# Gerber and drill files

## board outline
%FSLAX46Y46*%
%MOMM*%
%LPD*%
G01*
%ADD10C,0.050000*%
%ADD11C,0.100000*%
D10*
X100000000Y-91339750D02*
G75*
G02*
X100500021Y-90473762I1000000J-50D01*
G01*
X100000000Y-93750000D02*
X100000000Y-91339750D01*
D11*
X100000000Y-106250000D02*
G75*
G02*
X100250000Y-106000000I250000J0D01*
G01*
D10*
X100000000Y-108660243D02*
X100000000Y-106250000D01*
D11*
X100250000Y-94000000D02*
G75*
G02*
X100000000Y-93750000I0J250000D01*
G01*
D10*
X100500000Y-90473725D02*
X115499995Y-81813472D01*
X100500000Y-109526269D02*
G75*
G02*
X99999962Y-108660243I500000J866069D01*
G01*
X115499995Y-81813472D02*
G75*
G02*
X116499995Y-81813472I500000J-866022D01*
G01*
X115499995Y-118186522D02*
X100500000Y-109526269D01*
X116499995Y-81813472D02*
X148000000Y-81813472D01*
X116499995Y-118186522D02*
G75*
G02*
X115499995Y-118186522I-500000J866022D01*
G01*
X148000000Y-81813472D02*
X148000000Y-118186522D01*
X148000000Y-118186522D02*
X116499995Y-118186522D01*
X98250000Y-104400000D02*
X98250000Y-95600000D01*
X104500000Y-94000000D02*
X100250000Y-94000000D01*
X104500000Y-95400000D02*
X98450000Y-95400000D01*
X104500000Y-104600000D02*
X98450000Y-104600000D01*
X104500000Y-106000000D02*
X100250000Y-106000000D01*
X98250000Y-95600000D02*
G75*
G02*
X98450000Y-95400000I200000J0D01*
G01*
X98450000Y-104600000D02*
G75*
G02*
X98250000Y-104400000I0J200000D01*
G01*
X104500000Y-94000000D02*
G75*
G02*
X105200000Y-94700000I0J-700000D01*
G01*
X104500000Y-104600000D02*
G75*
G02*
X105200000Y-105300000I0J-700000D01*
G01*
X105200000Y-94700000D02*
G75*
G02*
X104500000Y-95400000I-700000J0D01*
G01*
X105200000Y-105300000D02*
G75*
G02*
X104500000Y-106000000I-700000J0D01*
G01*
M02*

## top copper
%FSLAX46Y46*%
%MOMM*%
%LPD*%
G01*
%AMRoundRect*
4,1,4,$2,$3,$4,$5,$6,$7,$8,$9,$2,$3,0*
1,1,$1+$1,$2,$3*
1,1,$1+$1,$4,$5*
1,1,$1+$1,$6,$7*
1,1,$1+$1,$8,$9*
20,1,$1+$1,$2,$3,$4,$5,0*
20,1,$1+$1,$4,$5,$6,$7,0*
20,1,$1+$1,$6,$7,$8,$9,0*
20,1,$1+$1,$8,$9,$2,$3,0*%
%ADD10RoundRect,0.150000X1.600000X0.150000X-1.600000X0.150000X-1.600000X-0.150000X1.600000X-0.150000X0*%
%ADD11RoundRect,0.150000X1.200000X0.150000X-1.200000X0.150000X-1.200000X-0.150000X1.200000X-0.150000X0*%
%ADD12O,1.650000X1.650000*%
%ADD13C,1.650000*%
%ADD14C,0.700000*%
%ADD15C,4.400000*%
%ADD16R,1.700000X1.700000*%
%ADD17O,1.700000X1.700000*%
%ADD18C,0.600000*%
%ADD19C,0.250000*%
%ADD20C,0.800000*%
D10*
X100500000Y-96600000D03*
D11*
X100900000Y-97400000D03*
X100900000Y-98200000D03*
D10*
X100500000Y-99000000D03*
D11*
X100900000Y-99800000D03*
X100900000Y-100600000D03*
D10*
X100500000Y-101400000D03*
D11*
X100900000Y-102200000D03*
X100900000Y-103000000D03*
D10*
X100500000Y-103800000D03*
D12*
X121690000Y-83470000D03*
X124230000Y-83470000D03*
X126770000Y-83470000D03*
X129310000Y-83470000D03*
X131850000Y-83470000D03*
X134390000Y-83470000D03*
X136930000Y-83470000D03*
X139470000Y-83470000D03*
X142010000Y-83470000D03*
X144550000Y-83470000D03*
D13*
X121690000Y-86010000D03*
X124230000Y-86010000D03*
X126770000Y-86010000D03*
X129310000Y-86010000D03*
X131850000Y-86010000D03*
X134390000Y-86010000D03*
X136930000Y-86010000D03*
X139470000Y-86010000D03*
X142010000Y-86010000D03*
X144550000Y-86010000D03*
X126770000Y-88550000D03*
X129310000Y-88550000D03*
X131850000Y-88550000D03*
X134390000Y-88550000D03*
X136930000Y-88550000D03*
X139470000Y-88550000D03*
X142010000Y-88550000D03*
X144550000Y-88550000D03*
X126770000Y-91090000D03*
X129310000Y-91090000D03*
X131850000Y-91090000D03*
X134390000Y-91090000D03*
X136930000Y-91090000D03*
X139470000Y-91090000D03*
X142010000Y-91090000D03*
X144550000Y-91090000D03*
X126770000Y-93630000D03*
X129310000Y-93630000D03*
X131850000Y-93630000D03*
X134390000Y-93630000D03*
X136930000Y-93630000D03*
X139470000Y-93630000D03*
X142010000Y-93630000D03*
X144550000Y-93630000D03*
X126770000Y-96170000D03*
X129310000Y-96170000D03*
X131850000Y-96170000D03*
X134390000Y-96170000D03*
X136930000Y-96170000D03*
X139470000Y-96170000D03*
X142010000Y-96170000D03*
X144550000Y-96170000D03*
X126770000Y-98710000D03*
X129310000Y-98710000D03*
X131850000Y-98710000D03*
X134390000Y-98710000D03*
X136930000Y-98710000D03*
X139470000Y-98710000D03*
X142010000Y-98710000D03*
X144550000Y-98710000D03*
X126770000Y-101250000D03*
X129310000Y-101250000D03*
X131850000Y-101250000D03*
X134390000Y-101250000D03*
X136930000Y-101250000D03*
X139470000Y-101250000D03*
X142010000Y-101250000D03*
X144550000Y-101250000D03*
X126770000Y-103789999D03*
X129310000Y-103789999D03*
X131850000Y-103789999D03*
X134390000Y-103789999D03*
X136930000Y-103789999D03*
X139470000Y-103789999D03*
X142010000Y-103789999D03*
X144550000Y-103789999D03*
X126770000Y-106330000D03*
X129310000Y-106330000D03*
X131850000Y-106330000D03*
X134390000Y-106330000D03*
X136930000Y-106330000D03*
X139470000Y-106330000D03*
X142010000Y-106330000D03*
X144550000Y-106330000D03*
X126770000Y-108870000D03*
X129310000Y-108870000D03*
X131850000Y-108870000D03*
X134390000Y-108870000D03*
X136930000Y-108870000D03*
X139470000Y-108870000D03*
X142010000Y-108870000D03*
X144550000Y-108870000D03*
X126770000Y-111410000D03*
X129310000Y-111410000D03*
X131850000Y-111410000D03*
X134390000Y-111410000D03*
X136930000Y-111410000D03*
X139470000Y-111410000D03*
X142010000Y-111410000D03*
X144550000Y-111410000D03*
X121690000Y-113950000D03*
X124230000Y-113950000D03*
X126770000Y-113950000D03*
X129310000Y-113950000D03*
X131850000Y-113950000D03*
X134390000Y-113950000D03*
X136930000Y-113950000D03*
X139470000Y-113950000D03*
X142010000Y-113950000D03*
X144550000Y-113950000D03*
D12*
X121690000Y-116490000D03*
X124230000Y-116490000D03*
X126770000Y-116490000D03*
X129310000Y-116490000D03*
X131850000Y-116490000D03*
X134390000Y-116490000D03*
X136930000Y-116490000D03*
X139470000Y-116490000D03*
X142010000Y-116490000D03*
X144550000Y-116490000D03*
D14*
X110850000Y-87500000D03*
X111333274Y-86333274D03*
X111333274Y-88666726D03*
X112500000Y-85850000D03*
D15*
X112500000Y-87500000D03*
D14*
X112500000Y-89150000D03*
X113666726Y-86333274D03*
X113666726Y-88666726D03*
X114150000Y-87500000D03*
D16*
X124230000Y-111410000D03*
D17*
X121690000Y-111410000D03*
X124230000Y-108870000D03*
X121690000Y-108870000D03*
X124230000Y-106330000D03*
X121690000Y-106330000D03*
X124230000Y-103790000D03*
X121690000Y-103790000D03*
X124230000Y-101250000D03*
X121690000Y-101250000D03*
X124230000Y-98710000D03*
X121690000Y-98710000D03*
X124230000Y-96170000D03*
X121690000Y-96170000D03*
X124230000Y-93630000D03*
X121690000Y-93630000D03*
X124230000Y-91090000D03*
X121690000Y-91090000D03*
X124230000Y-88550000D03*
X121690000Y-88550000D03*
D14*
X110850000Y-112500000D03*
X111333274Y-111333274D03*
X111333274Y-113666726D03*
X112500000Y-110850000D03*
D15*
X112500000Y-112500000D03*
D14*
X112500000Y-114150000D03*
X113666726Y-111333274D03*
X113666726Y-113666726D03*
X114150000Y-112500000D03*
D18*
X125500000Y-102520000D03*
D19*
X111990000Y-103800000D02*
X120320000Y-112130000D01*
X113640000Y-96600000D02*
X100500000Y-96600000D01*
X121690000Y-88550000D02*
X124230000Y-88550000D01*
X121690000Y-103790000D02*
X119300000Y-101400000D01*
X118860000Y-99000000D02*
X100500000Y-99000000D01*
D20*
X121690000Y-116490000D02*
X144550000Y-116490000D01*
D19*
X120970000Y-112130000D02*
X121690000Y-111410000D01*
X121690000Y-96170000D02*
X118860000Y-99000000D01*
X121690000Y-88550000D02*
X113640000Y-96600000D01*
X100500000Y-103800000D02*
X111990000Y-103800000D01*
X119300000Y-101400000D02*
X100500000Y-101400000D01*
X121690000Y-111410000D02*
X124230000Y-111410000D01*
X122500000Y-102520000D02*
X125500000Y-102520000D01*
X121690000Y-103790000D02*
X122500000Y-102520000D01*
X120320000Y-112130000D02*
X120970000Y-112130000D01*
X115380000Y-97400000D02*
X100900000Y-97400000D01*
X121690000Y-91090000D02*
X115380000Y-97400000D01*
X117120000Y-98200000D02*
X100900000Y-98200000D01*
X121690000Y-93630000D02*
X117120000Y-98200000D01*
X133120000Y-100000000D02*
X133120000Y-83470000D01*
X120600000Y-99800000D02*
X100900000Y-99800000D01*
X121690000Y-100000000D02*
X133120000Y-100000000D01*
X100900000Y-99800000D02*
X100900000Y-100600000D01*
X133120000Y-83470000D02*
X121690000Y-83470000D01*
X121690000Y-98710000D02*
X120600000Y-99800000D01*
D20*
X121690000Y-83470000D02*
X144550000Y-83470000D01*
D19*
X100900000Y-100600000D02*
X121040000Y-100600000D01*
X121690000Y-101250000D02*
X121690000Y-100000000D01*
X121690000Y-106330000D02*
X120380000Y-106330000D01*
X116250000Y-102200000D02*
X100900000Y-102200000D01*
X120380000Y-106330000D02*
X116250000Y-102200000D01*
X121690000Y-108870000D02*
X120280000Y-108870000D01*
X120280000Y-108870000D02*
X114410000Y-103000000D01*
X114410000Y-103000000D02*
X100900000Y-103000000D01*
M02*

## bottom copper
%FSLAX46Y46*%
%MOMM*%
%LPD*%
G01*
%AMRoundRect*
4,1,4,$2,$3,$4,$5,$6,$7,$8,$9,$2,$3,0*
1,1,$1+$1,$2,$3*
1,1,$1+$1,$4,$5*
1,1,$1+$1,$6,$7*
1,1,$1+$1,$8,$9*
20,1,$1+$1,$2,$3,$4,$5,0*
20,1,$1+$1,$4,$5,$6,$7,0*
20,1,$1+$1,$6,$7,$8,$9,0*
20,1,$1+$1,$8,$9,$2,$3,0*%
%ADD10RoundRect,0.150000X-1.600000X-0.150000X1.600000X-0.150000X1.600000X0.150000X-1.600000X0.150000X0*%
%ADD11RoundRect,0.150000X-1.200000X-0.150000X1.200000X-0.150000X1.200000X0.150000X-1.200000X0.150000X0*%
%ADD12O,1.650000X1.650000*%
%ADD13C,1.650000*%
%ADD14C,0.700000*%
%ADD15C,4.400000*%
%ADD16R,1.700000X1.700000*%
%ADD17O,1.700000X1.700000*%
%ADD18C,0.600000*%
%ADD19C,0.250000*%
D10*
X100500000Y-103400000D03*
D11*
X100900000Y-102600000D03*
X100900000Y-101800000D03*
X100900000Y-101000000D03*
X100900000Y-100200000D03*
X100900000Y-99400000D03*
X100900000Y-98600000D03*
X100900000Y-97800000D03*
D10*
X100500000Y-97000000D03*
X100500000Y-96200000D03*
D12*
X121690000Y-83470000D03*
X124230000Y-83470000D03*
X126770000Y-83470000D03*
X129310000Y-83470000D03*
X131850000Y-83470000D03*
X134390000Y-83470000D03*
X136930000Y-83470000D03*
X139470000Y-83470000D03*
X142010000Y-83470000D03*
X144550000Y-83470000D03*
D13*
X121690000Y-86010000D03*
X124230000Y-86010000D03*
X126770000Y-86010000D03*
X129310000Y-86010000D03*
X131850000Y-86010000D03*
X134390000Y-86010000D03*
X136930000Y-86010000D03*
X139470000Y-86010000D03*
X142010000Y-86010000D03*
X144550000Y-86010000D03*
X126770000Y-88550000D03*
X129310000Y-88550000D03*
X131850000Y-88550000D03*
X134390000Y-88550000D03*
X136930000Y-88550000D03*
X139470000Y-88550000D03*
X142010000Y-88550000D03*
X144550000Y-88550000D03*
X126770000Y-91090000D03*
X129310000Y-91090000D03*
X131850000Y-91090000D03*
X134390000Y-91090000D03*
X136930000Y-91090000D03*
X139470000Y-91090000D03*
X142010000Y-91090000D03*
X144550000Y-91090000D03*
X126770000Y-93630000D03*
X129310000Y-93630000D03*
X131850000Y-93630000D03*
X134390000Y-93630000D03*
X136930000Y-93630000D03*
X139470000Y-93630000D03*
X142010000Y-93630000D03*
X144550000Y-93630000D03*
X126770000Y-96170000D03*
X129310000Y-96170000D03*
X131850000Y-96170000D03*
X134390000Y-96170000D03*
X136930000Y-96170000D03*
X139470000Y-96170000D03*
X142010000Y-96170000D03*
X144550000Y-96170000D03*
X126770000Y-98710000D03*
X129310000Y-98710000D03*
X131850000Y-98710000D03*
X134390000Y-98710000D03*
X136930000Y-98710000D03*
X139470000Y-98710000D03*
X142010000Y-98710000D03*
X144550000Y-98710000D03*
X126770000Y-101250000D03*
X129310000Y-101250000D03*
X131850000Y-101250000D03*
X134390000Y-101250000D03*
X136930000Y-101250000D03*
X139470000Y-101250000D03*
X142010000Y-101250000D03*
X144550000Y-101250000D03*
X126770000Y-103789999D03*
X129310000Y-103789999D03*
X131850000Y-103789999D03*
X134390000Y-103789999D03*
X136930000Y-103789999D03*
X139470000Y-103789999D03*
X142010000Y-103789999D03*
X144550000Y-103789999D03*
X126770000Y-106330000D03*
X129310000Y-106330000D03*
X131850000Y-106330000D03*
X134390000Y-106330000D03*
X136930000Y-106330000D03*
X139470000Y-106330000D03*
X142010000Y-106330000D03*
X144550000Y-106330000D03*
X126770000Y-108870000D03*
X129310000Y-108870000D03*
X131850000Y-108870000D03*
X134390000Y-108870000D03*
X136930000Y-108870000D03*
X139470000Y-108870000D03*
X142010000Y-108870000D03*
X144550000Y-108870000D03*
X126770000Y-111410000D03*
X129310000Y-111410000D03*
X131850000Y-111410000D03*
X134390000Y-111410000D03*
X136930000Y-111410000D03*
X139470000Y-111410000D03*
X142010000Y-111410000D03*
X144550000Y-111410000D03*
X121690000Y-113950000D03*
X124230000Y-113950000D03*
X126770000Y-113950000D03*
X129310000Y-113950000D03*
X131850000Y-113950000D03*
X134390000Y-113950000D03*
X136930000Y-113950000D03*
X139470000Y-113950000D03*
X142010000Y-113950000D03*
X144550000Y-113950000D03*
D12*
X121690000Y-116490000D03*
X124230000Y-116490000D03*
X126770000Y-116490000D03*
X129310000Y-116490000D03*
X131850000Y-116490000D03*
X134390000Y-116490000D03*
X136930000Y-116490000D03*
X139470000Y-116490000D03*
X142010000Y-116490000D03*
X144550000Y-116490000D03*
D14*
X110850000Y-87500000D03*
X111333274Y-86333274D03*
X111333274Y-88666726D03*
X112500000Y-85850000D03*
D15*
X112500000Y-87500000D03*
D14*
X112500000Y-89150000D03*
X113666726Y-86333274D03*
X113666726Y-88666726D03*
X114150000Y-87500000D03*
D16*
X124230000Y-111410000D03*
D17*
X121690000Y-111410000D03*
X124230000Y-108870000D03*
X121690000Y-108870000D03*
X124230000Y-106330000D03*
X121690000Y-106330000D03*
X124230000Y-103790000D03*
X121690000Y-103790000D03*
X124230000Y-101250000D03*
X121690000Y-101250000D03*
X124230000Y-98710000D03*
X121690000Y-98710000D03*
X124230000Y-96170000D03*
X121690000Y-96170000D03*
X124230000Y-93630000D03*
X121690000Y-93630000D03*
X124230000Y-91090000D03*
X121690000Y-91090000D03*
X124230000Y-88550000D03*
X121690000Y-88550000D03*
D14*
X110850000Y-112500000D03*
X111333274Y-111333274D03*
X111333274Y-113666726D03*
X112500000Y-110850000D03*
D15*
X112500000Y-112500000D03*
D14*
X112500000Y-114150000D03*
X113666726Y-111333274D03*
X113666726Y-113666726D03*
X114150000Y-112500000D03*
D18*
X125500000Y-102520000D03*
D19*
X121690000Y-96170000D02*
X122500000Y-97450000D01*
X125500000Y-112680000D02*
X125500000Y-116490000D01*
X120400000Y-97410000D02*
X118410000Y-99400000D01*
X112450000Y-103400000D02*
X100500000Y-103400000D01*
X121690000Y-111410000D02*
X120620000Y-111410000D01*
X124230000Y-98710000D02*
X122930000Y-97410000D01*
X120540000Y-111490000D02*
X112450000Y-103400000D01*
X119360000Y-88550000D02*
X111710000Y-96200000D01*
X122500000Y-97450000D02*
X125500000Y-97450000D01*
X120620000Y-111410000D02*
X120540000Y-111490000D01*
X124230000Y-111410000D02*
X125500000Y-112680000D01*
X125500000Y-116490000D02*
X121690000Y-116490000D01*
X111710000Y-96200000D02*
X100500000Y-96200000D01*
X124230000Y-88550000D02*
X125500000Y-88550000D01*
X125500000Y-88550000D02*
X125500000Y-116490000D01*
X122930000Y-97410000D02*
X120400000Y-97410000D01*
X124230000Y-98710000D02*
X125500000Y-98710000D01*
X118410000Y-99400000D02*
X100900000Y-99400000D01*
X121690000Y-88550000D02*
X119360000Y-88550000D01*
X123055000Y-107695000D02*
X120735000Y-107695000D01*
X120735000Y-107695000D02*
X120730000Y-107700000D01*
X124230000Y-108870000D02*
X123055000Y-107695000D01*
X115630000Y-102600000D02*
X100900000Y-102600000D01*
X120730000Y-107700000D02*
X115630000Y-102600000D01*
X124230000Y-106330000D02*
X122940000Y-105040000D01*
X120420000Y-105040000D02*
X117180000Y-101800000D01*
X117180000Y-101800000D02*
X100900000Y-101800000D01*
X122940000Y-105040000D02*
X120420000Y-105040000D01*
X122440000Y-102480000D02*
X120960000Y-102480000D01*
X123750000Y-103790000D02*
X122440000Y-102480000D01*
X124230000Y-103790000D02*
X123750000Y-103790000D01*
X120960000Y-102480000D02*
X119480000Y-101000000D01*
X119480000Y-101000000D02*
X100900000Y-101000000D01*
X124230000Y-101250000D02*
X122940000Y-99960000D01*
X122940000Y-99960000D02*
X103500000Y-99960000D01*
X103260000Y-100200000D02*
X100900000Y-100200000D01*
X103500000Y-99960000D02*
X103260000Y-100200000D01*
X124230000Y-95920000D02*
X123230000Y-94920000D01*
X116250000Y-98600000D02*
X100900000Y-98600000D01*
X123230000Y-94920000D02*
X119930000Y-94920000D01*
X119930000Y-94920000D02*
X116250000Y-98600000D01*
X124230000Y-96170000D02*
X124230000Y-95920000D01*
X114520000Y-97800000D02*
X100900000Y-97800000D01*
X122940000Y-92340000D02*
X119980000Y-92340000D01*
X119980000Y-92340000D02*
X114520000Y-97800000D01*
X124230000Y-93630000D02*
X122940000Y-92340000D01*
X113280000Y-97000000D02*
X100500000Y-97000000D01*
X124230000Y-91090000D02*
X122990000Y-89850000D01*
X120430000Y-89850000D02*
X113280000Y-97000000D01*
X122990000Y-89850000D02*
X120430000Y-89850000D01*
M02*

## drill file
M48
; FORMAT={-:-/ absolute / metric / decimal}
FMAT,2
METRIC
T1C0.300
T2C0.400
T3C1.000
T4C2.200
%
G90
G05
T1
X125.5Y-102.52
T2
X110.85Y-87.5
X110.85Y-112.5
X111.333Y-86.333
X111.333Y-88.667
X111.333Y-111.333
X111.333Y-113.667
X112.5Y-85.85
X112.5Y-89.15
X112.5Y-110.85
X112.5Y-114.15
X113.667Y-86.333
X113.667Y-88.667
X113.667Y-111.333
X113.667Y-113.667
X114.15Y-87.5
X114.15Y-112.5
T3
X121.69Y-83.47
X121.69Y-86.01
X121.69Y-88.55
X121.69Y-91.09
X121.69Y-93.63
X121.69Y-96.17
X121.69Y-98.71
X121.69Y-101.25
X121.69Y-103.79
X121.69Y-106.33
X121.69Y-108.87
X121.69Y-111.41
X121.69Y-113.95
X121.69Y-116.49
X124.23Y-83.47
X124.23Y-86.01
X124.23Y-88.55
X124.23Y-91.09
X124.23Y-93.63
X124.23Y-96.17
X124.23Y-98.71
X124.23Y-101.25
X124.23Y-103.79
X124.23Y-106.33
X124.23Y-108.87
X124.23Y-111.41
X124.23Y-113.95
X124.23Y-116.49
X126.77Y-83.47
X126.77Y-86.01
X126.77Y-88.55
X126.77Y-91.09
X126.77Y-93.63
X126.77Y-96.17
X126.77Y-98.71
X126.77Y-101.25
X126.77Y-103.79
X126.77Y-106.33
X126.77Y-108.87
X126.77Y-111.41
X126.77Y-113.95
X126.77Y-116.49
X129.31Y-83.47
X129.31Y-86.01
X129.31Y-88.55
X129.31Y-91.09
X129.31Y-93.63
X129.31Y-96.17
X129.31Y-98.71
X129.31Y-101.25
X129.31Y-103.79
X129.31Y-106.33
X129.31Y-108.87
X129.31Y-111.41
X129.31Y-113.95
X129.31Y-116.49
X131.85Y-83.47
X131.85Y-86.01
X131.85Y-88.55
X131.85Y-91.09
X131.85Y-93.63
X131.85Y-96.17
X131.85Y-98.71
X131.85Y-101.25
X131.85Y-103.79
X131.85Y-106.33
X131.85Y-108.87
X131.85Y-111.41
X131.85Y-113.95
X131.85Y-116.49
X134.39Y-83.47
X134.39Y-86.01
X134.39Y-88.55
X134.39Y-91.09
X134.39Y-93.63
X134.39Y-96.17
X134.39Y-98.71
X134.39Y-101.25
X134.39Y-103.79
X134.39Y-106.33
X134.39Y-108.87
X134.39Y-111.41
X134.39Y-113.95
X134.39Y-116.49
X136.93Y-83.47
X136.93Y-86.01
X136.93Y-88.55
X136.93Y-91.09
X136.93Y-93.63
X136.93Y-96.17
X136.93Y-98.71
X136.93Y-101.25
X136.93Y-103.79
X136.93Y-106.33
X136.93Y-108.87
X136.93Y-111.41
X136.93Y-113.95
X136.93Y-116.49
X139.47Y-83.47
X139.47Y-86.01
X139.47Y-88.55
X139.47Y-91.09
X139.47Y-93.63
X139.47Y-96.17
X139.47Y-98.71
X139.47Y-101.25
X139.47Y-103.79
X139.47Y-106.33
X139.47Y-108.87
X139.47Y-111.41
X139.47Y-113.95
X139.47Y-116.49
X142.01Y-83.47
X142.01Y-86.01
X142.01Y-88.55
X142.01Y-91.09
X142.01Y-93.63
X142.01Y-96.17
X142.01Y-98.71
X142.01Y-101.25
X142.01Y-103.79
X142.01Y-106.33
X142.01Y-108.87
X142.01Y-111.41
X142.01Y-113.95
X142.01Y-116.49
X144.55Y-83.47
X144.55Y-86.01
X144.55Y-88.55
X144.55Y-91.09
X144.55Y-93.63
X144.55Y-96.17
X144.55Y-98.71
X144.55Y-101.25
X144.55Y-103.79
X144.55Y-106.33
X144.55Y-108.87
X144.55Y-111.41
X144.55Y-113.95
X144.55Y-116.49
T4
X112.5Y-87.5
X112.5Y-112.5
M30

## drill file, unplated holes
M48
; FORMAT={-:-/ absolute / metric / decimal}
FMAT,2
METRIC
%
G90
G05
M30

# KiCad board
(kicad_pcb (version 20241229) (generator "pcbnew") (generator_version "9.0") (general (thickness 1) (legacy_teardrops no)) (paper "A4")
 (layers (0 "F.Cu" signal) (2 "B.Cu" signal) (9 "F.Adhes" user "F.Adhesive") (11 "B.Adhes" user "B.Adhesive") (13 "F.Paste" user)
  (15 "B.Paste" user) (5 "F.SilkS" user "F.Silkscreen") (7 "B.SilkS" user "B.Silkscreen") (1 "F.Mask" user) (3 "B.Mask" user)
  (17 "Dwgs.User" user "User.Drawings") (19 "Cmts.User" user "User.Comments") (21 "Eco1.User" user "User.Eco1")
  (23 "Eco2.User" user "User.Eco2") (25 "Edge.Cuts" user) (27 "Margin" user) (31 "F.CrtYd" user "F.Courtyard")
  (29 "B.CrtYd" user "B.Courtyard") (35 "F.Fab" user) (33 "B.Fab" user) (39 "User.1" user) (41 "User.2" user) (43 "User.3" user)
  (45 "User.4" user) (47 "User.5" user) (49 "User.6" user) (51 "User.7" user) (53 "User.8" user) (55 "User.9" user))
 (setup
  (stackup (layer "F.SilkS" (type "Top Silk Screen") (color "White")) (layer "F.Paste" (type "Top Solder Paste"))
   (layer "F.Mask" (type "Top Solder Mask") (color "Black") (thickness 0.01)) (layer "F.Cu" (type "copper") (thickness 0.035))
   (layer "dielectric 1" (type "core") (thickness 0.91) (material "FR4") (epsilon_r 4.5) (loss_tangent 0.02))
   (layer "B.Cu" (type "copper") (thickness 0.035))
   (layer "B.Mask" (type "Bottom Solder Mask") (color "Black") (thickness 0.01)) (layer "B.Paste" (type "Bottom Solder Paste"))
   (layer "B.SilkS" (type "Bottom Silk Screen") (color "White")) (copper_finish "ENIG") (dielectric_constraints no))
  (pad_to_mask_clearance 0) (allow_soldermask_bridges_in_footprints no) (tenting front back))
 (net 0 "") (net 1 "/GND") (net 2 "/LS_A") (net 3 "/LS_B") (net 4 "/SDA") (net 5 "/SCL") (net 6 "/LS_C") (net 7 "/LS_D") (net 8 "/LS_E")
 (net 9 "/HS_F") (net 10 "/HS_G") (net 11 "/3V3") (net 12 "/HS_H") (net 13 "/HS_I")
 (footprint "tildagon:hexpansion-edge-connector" (layer "F.Cu") (at 98.25 100)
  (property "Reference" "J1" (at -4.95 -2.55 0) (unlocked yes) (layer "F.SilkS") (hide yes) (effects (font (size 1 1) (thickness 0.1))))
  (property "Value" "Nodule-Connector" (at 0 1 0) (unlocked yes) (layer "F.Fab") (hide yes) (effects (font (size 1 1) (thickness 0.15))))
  (fp_line (start 0 4.4) (end 0 -4.4) (stroke (width 0.05) (type solid)) (layer "Edge.Cuts"))
  (fp_line (start 6.25 -6) (end 2 -6) (stroke (width 0.05) (type solid)) (layer "Edge.Cuts"))
  (fp_line (start 6.25 -4.6) (end 0.2 -4.6) (stroke (width 0.05) (type solid)) (layer "Edge.Cuts"))
  (fp_line (start 6.25 4.6) (end 0.2 4.6) (stroke (width 0.05) (type solid)) (layer "Edge.Cuts"))
  (fp_line (start 6.25 6) (end 2 6) (stroke (width 0.05) (type solid)) (layer "Edge.Cuts"))
  (fp_arc (start 0 -4.4) (mid 0.058579 -4.541421) (end 0.2 -4.6) (stroke (width 0.05) (type default)) (layer "Edge.Cuts"))
  (fp_arc (start 0.2 4.6) (mid 0.058579 4.541421) (end 0 4.4) (stroke (width 0.05) (type default)) (layer "Edge.Cuts"))
  (fp_arc (start 6.25 -6) (mid 6.744975 -5.794975) (end 6.95 -5.3) (stroke (width 0.05) (type default)) (layer "Edge.Cuts"))
  (fp_arc (start 6.25 4.6) (mid 6.744975 4.805025) (end 6.95 5.3) (stroke (width 0.05) (type default)) (layer "Edge.Cuts"))
  (fp_arc (start 6.95 -5.3) (mid 6.744975 -4.805025) (end 6.25 -4.6) (stroke (width 0.05) (type default)) (layer "Edge.Cuts"))
  (fp_arc (start 6.95 5.3) (mid 6.744975 5.794975) (end 6.25 6) (stroke (width 0.05) (type default)) (layer "Edge.Cuts"))
  (pad "1" smd roundrect (at 2.25 3.4) (size 3.5 0.6) (layers "B.Cu" "B.Mask") (roundrect_rratio 0.25) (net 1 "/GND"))
  (pad "2" smd roundrect (at 2.65 2.6) (size 2.7 0.6) (layers "B.Cu" "B.Mask") (roundrect_rratio 0.25) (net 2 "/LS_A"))
  (pad "3" smd roundrect (at 2.65 1.8) (size 2.7 0.6) (layers "B.Cu" "B.Mask") (roundrect_rratio 0.25) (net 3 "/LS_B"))
  (pad "4" smd roundrect (at 2.65 1) (size 2.7 0.6) (layers "B.Cu" "B.Mask") (roundrect_rratio 0.25) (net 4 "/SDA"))
  (pad "5" smd roundrect (at 2.65 0.2) (size 2.7 0.6) (layers "B.Cu" "B.Mask") (roundrect_rratio 0.25) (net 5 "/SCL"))
  (pad "6" smd roundrect (at 2.65 -0.6) (size 2.7 0.6) (layers "B.Cu" "B.Mask") (roundrect_rratio 0.25) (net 1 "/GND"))
  (pad "7" smd roundrect (at 2.65 -1.4) (size 2.7 0.6) (layers "B.Cu" "B.Mask") (roundrect_rratio 0.25) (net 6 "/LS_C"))
  (pad "8" smd roundrect (at 2.65 -2.2) (size 2.7 0.6) (layers "B.Cu" "B.Mask") (roundrect_rratio 0.25) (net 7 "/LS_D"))
  (pad "9" smd roundrect (at 2.25 -3) (size 3.5 0.6) (layers "B.Cu" "B.Mask") (roundrect_rratio 0.25) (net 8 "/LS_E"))
  (pad "10" smd roundrect (at 2.25 -3.8) (size 3.5 0.6) (layers "B.Cu" "B.Mask") (roundrect_rratio 0.25) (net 1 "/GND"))
  (pad "11" smd roundrect (at 2.25 -3.4 180) (size 3.5 0.6) (layers "F.Cu" "F.Mask") (roundrect_rratio 0.25) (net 1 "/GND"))
  (pad "12" smd roundrect (at 2.65 -2.6 180) (size 2.7 0.6) (layers "F.Cu" "F.Mask") (roundrect_rratio 0.25) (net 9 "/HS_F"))
  (pad "13" smd roundrect (at 2.65 -1.8 180) (size 2.7 0.6) (layers "F.Cu" "F.Mask") (roundrect_rratio 0.25) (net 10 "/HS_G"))
  (pad "14" smd roundrect (at 2.25 -1 180) (size 3.5 0.6) (layers "F.Cu" "F.Mask") (roundrect_rratio 0.25) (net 1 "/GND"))
  (pad "15" smd roundrect (at 2.65 -0.2 180) (size 2.7 0.6) (layers "F.Cu" "F.Mask") (roundrect_rratio 0.25) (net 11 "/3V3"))
  (pad "16" smd roundrect (at 2.65 0.6 180) (size 2.7 0.6) (layers "F.Cu" "F.Mask") (roundrect_rratio 0.25) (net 11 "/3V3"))
  (pad "17" smd roundrect (at 2.25 1.4 180) (size 3.5 0.6) (layers "F.Cu" "F.Mask") (roundrect_rratio 0.25) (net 1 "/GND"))
  (pad "18" smd roundrect (at 2.65 2.2 180) (size 2.7 0.6) (layers "F.Cu" "F.Mask") (roundrect_rratio 0.25) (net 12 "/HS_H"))
  (pad "19" smd roundrect (at 2.65 3 180) (size 2.7 0.6) (layers "F.Cu" "F.Mask") (roundrect_rratio 0.25) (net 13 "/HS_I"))
  (pad "20" smd roundrect (at 2.25 3.8 180) (size 3.5 0.6) (layers "F.Cu" "F.Mask") (roundrect_rratio 0.25) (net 1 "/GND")))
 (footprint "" (layer "F.Cu") (at 0 0)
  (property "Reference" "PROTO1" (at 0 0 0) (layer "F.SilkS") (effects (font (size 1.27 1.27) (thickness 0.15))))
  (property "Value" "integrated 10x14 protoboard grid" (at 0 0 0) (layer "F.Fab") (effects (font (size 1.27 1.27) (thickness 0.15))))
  (pad "1" thru_hole oval (at 121.69 83.47) (size 1.65 1.65) (drill 1) (layers "*.Cu" "*.Mask") (remove_unused_layers no) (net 11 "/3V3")
   (thermal_bridge_angle 45))
  (pad "2" thru_hole oval (at 124.23 83.47) (size 1.65 1.65) (drill 1) (layers "*.Cu" "*.Mask") (remove_unused_layers no) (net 11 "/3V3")
   (thermal_bridge_angle 45))
  (pad "3" thru_hole oval (at 126.77 83.47) (size 1.65 1.65) (drill 1) (layers "*.Cu" "*.Mask") (remove_unused_layers no) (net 11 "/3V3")
   (thermal_bridge_angle 45))
  (pad "4" thru_hole oval (at 129.31 83.47) (size 1.65 1.65) (drill 1) (layers "*.Cu" "*.Mask") (remove_unused_layers no) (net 11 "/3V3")
   (thermal_bridge_angle 45))
  (pad "5" thru_hole oval (at 131.85 83.47) (size 1.65 1.65) (drill 1) (layers "*.Cu" "*.Mask") (remove_unused_layers no) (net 11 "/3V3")
   (thermal_bridge_angle 45))
  (pad "6" thru_hole oval (at 134.39 83.47) (size 1.65 1.65) (drill 1) (layers "*.Cu" "*.Mask") (remove_unused_layers no) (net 11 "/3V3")
   (thermal_bridge_angle 45))
  (pad "7" thru_hole oval (at 136.93 83.47) (size 1.65 1.65) (drill 1) (layers "*.Cu" "*.Mask") (remove_unused_layers no) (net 11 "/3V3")
   (thermal_bridge_angle 45))
  (pad "8" thru_hole oval (at 139.47 83.47) (size 1.65 1.65) (drill 1) (layers "*.Cu" "*.Mask") (remove_unused_layers no) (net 11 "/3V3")
   (thermal_bridge_angle 45))
  (pad "9" thru_hole oval (at 142.01 83.47) (size 1.65 1.65) (drill 1) (layers "*.Cu" "*.Mask") (remove_unused_layers no) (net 11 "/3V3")
   (thermal_bridge_angle 45))
  (pad "10" thru_hole oval (at 144.55 83.47) (size 1.65 1.65) (drill 1) (layers "*.Cu" "*.Mask") (remove_unused_layers no) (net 11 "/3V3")
   (thermal_bridge_angle 45))
  (pad "11" thru_hole circle (at 121.69 86.01) (size 1.65 1.65) (drill 1) (layers "*.Cu" "*.Mask") (remove_unused_layers no))
  (pad "12" thru_hole circle (at 124.23 86.01) (size 1.65 1.65) (drill 1) (layers "*.Cu" "*.Mask") (remove_unused_layers no))
  (pad "13" thru_hole circle (at 126.77 86.01) (size 1.65 1.65) (drill 1) (layers "*.Cu" "*.Mask") (remove_unused_layers no))
  (pad "14" thru_hole circle (at 129.31 86.01) (size 1.65 1.65) (drill 1) (layers "*.Cu" "*.Mask") (remove_unused_layers no))
  (pad "15" thru_hole circle (at 131.85 86.01) (size 1.65 1.65) (drill 1) (layers "*.Cu" "*.Mask") (remove_unused_layers no))
  (pad "16" thru_hole circle (at 134.39 86.01) (size 1.65 1.65) (drill 1) (layers "*.Cu" "*.Mask") (remove_unused_layers no))
  (pad "17" thru_hole circle (at 136.93 86.01) (size 1.65 1.65) (drill 1) (layers "*.Cu" "*.Mask") (remove_unused_layers no))
  (pad "18" thru_hole circle (at 139.47 86.01) (size 1.65 1.65) (drill 1) (layers "*.Cu" "*.Mask") (remove_unused_layers no))
  (pad "19" thru_hole circle (at 142.01 86.01) (size 1.65 1.65) (drill 1) (layers "*.Cu" "*.Mask") (remove_unused_layers no))
  (pad "20" thru_hole circle (at 144.55 86.01) (size 1.65 1.65) (drill 1) (layers "*.Cu" "*.Mask") (remove_unused_layers no))
  (pad "21" thru_hole circle (at 126.77 88.55) (size 1.65 1.65) (drill 1) (layers "*.Cu" "*.Mask") (remove_unused_layers no))
  (pad "22" thru_hole circle (at 129.31 88.55) (size 1.65 1.65) (drill 1) (layers "*.Cu" "*.Mask") (remove_unused_layers no))
  (pad "23" thru_hole circle (at 131.85 88.55) (size 1.65 1.65) (drill 1) (layers "*.Cu" "*.Mask") (remove_unused_layers no))
  (pad "24" thru_hole circle (at 134.39 88.55) (size 1.65 1.65) (drill 1) (layers "*.Cu" "*.Mask") (remove_unused_layers no))
  (pad "25" thru_hole circle (at 136.93 88.55) (size 1.65 1.65) (drill 1) (layers "*.Cu" "*.Mask") (remove_unused_layers no))
  (pad "26" thru_hole circle (at 139.47 88.55) (size 1.65 1.65) (drill 1) (layers "*.Cu" "*.Mask") (remove_unused_layers no))
  (pad "27" thru_hole circle (at 142.01 88.55) (size 1.65 1.65) (drill 1) (layers "*.Cu" "*.Mask") (remove_unused_layers no))
  (pad "28" thru_hole circle (at 144.55 88.55) (size 1.65 1.65) (drill 1) (layers "*.Cu" "*.Mask") (remove_unused_layers no))
  (pad "29" thru_hole circle (at 126.77 91.09) (size 1.65 1.65) (drill 1) (layers "*.Cu" "*.Mask") (remove_unused_layers no))
  (pad "30" thru_hole circle (at 129.31 91.09) (size 1.65 1.65) (drill 1) (layers "*.Cu" "*.Mask") (remove_unused_layers no))
  (pad "31" thru_hole circle (at 131.85 91.09) (size 1.65 1.65) (drill 1) (layers "*.Cu" "*.Mask") (remove_unused_layers no))
  (pad "32" thru_hole circle (at 134.39 91.09) (size 1.65 1.65) (drill 1) (layers "*.Cu" "*.Mask") (remove_unused_layers no))
  (pad "33" thru_hole circle (at 136.93 91.09) (size 1.65 1.65) (drill 1) (layers "*.Cu" "*.Mask") (remove_unused_layers no))
  (pad "34" thru_hole circle (at 139.47 91.09) (size 1.65 1.65) (drill 1) (layers "*.Cu" "*.Mask") (remove_unused_layers no))
  (pad "35" thru_hole circle (at 142.01 91.09) (size 1.65 1.65) (drill 1) (layers "*.Cu" "*.Mask") (remove_unused_layers no))
  (pad "36" thru_hole circle (at 144.55 91.09) (size 1.65 1.65) (drill 1) (layers "*.Cu" "*.Mask") (remove_unused_layers no))
  (pad "37" thru_hole circle (at 126.77 93.63) (size 1.65 1.65) (drill 1) (layers "*.Cu" "*.Mask") (remove_unused_layers no))
  (pad "38" thru_hole circle (at 129.31 93.63) (size 1.65 1.65) (drill 1) (layers "*.Cu" "*.Mask") (remove_unused_layers no))
  (pad "39" thru_hole circle (at 131.85 93.63) (size 1.65 1.65) (drill 1) (layers "*.Cu" "*.Mask") (remove_unused_layers no))
  (pad "40" thru_hole circle (at 134.39 93.63) (size 1.65 1.65) (drill 1) (layers "*.Cu" "*.Mask") (remove_unused_layers no))
  (pad "41" thru_hole circle (at 136.93 93.63) (size 1.65 1.65) (drill 1) (layers "*.Cu" "*.Mask") (remove_unused_layers no))
  (pad "42" thru_hole circle (at 139.47 93.63) (size 1.65 1.65) (drill 1) (layers "*.Cu" "*.Mask") (remove_unused_layers no))
  (pad "43" thru_hole circle (at 142.01 93.63) (size 1.65 1.65) (drill 1) (layers "*.Cu" "*.Mask") (remove_unused_layers no))
  (pad "44" thru_hole circle (at 144.55 93.63) (size 1.65 1.65) (drill 1) (layers "*.Cu" "*.Mask") (remove_unused_layers no))
  (pad "45" thru_hole circle (at 126.77 96.17) (size 1.65 1.65) (drill 1) (layers "*.Cu" "*.Mask") (remove_unused_layers no))
  (pad "46" thru_hole circle (at 129.31 96.17) (size 1.65 1.65) (drill 1) (layers "*.Cu" "*.Mask") (remove_unused_layers no))
  (pad "47" thru_hole circle (at 131.85 96.17) (size 1.65 1.65) (drill 1) (layers "*.Cu" "*.Mask") (remove_unused_layers no))
  (pad "48" thru_hole circle (at 134.39 96.17) (size 1.65 1.65) (drill 1) (layers "*.Cu" "*.Mask") (remove_unused_layers no))
  (pad "49" thru_hole circle (at 136.93 96.17) (size 1.65 1.65) (drill 1) (layers "*.Cu" "*.Mask") (remove_unused_layers no))
  (pad "50" thru_hole circle (at 139.47 96.17) (size 1.65 1.65) (drill 1) (layers "*.Cu" "*.Mask") (remove_unused_layers no))
  (pad "51" thru_hole circle (at 142.01 96.17) (size 1.65 1.65) (drill 1) (layers "*.Cu" "*.Mask") (remove_unused_layers no))
  (pad "52" thru_hole circle (at 144.55 96.17) (size 1.65 1.65) (drill 1) (layers "*.Cu" "*.Mask") (remove_unused_layers no))
  (pad "53" thru_hole circle (at 126.77 98.71) (size 1.65 1.65) (drill 1) (layers "*.Cu" "*.Mask") (remove_unused_layers no))
  (pad "54" thru_hole circle (at 129.31 98.71) (size 1.65 1.65) (drill 1) (layers "*.Cu" "*.Mask") (remove_unused_layers no))
  (pad "55" thru_hole circle (at 131.85 98.71) (size 1.65 1.65) (drill 1) (layers "*.Cu" "*.Mask") (remove_unused_layers no))
  (pad "56" thru_hole circle (at 134.39 98.71) (size 1.65 1.65) (drill 1) (layers "*.Cu" "*.Mask") (remove_unused_layers no))
  (pad "57" thru_hole circle (at 136.93 98.71) (size 1.65 1.65) (drill 1) (layers "*.Cu" "*.Mask") (remove_unused_layers no))
  (pad "58" thru_hole circle (at 139.47 98.71) (size 1.65 1.65) (drill 1) (layers "*.Cu" "*.Mask") (remove_unused_layers no))
  (pad "59" thru_hole circle (at 142.01 98.71) (size 1.65 1.65) (drill 1) (layers "*.Cu" "*.Mask") (remove_unused_layers no))
  (pad "60" thru_hole circle (at 144.55 98.71) (size 1.65 1.65) (drill 1) (layers "*.Cu" "*.Mask") (remove_unused_layers no))
  (pad "61" thru_hole circle (at 126.77 101.25) (size 1.65 1.65) (drill 1) (layers "*.Cu" "*.Mask") (remove_unused_layers no))
  (pad "62" thru_hole circle (at 129.31 101.25) (size 1.65 1.65) (drill 1) (layers "*.Cu" "*.Mask") (remove_unused_layers no))
  (pad "63" thru_hole circle (at 131.85 101.25) (size 1.65 1.65) (drill 1) (layers "*.Cu" "*.Mask") (remove_unused_layers no))
  (pad "64" thru_hole circle (at 134.39 101.25) (size 1.65 1.65) (drill 1) (layers "*.Cu" "*.Mask") (remove_unused_layers no))
  (pad "65" thru_hole circle (at 136.93 101.25) (size 1.65 1.65) (drill 1) (layers "*.Cu" "*.Mask") (remove_unused_layers no))
  (pad "66" thru_hole circle (at 139.47 101.25) (size 1.65 1.65) (drill 1) (layers "*.Cu" "*.Mask") (remove_unused_layers no))
  (pad "67" thru_hole circle (at 142.01 101.25) (size 1.65 1.65) (drill 1) (layers "*.Cu" "*.Mask") (remove_unused_layers no))
  (pad "68" thru_hole circle (at 144.55 101.25) (size 1.65 1.65) (drill 1) (layers "*.Cu" "*.Mask") (remove_unused_layers no))
  (pad "69" thru_hole circle (at 126.77 103.789999) (size 1.65 1.65) (drill 1) (layers "*.Cu" "*.Mask") (remove_unused_layers no))
  (pad "70" thru_hole circle (at 129.31 103.789999) (size 1.65 1.65) (drill 1) (layers "*.Cu" "*.Mask") (remove_unused_layers no))
  (pad "71" thru_hole circle (at 131.85 103.789999) (size 1.65 1.65) (drill 1) (layers "*.Cu" "*.Mask") (remove_unused_layers no))
  (pad "72" thru_hole circle (at 134.39 103.789999) (size 1.65 1.65) (drill 1) (layers "*.Cu" "*.Mask") (remove_unused_layers no))
  (pad "73" thru_hole circle (at 136.93 103.789999) (size 1.65 1.65) (drill 1) (layers "*.Cu" "*.Mask") (remove_unused_layers no))
  (pad "74" thru_hole circle (at 139.47 103.789999) (size 1.65 1.65) (drill 1) (layers "*.Cu" "*.Mask") (remove_unused_layers no))
  (pad "75" thru_hole circle (at 142.01 103.789999) (size 1.65 1.65) (drill 1) (layers "*.Cu" "*.Mask") (remove_unused_layers no))
  (pad "76" thru_hole circle (at 144.55 103.789999) (size 1.65 1.65) (drill 1) (layers "*.Cu" "*.Mask") (remove_unused_layers no))
  (pad "77" thru_hole circle (at 126.77 106.33) (size 1.65 1.65) (drill 1) (layers "*.Cu" "*.Mask") (remove_unused_layers no))
  (pad "78" thru_hole circle (at 129.31 106.33) (size 1.65 1.65) (drill 1) (layers "*.Cu" "*.Mask") (remove_unused_layers no))
  (pad "79" thru_hole circle (at 131.85 106.33) (size 1.65 1.65) (drill 1) (layers "*.Cu" "*.Mask") (remove_unused_layers no))
  (pad "80" thru_hole circle (at 134.39 106.33) (size 1.65 1.65) (drill 1) (layers "*.Cu" "*.Mask") (remove_unused_layers no))
  (pad "81" thru_hole circle (at 136.93 106.33) (size 1.65 1.65) (drill 1) (layers "*.Cu" "*.Mask") (remove_unused_layers no))
  (pad "82" thru_hole circle (at 139.47 106.33) (size 1.65 1.65) (drill 1) (layers "*.Cu" "*.Mask") (remove_unused_layers no))
  (pad "83" thru_hole circle (at 142.01 106.33) (size 1.65 1.65) (drill 1) (layers "*.Cu" "*.Mask") (remove_unused_layers no))
  (pad "84" thru_hole circle (at 144.55 106.33) (size 1.65 1.65) (drill 1) (layers "*.Cu" "*.Mask") (remove_unused_layers no))
  (pad "85" thru_hole circle (at 126.77 108.87) (size 1.65 1.65) (drill 1) (layers "*.Cu" "*.Mask") (remove_unused_layers no))
  (pad "86" thru_hole circle (at 129.31 108.87) (size 1.65 1.65) (drill 1) (layers "*.Cu" "*.Mask") (remove_unused_layers no))
  (pad "87" thru_hole circle (at 131.85 108.87) (size 1.65 1.65) (drill 1) (layers "*.Cu" "*.Mask") (remove_unused_layers no))
  (pad "88" thru_hole circle (at 134.39 108.87) (size 1.65 1.65) (drill 1) (layers "*.Cu" "*.Mask") (remove_unused_layers no))
  (pad "89" thru_hole circle (at 136.93 108.87) (size 1.65 1.65) (drill 1) (layers "*.Cu" "*.Mask") (remove_unused_layers no))
  (pad "90" thru_hole circle (at 139.47 108.87) (size 1.65 1.65) (drill 1) (layers "*.Cu" "*.Mask") (remove_unused_layers no))
  (pad "91" thru_hole circle (at 142.01 108.87) (size 1.65 1.65) (drill 1) (layers "*.Cu" "*.Mask") (remove_unused_layers no))
  (pad "92" thru_hole circle (at 144.55 108.87) (size 1.65 1.65) (drill 1) (layers "*.Cu" "*.Mask") (remove_unused_layers no))
  (pad "93" thru_hole circle (at 126.77 111.41) (size 1.65 1.65) (drill 1) (layers "*.Cu" "*.Mask") (remove_unused_layers no))
  (pad "94" thru_hole circle (at 129.31 111.41) (size 1.65 1.65) (drill 1) (layers "*.Cu" "*.Mask") (remove_unused_layers no))
  (pad "95" thru_hole circle (at 131.85 111.41) (size 1.65 1.65) (drill 1) (layers "*.Cu" "*.Mask") (remove_unused_layers no))
  (pad "96" thru_hole circle (at 134.39 111.41) (size 1.65 1.65) (drill 1) (layers "*.Cu" "*.Mask") (remove_unused_layers no))
  (pad "97" thru_hole circle (at 136.93 111.41) (size 1.65 1.65) (drill 1) (layers "*.Cu" "*.Mask") (remove_unused_layers no))
  (pad "98" thru_hole circle (at 139.47 111.41) (size 1.65 1.65) (drill 1) (layers "*.Cu" "*.Mask") (remove_unused_layers no))
  (pad "99" thru_hole circle (at 142.01 111.41) (size 1.65 1.65) (drill 1) (layers "*.Cu" "*.Mask") (remove_unused_layers no))
  (pad "100" thru_hole circle (at 144.55 111.41) (size 1.65 1.65) (drill 1) (layers "*.Cu" "*.Mask") (remove_unused_layers no))
  (pad "101" thru_hole circle (at 121.69 113.95) (size 1.65 1.65) (drill 1) (layers "*.Cu" "*.Mask") (remove_unused_layers no))
  (pad "102" thru_hole circle (at 124.23 113.95) (size 1.65 1.65) (drill 1) (layers "*.Cu" "*.Mask") (remove_unused_layers no))
  (pad "103" thru_hole circle (at 126.77 113.95) (size 1.65 1.65) (drill 1) (layers "*.Cu" "*.Mask") (remove_unused_layers no))
  (pad "104" thru_hole circle (at 129.31 113.95) (size 1.65 1.65) (drill 1) (layers "*.Cu" "*.Mask") (remove_unused_layers no))
  (pad "105" thru_hole circle (at 131.85 113.95) (size 1.65 1.65) (drill 1) (layers "*.Cu" "*.Mask") (remove_unused_layers no))
  (pad "106" thru_hole circle (at 134.39 113.95) (size 1.65 1.65) (drill 1) (layers "*.Cu" "*.Mask") (remove_unused_layers no))
  (pad "107" thru_hole circle (at 136.93 113.95) (size 1.65 1.65) (drill 1) (layers "*.Cu" "*.Mask") (remove_unused_layers no))
  (pad "108" thru_hole circle (at 139.47 113.95) (size 1.65 1.65) (drill 1) (layers "*.Cu" "*.Mask") (remove_unused_layers no))
  (pad "109" thru_hole circle (at 142.01 113.95) (size 1.65 1.65) (drill 1) (layers "*.Cu" "*.Mask") (remove_unused_layers no))
  (pad "110" thru_hole circle (at 144.55 113.95) (size 1.65 1.65) (drill 1) (layers "*.Cu" "*.Mask") (remove_unused_layers no))
  (pad "111" thru_hole oval (at 121.69 116.49) (size 1.65 1.65) (drill 1) (layers "*.Cu" "*.Mask") (remove_unused_layers no) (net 1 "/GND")
   (thermal_bridge_angle 45))
  (pad "112" thru_hole oval (at 124.23 116.49) (size 1.65 1.65) (drill 1) (layers "*.Cu" "*.Mask") (remove_unused_layers no) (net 1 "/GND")
   (thermal_bridge_angle 45))
  (pad "113" thru_hole oval (at 126.77 116.49) (size 1.65 1.65) (drill 1) (layers "*.Cu" "*.Mask") (remove_unused_layers no) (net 1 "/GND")
   (thermal_bridge_angle 45))
  (pad "114" thru_hole oval (at 129.31 116.49) (size 1.65 1.65) (drill 1) (layers "*.Cu" "*.Mask") (remove_unused_layers no) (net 1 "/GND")
   (thermal_bridge_angle 45))
  (pad "115" thru_hole oval (at 131.85 116.49) (size 1.65 1.65) (drill 1) (layers "*.Cu" "*.Mask") (remove_unused_layers no) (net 1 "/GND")
   (thermal_bridge_angle 45))
  (pad "116" thru_hole oval (at 134.39 116.49) (size 1.65 1.65) (drill 1) (layers "*.Cu" "*.Mask") (remove_unused_layers no) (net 1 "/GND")
   (thermal_bridge_angle 45))
  (pad "117" thru_hole oval (at 136.93 116.49) (size 1.65 1.65) (drill 1) (layers "*.Cu" "*.Mask") (remove_unused_layers no) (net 1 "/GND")
   (thermal_bridge_angle 45))
  (pad "118" thru_hole oval (at 139.47 116.49) (size 1.65 1.65) (drill 1) (layers "*.Cu" "*.Mask") (remove_unused_layers no) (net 1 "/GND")
   (thermal_bridge_angle 45))
  (pad "119" thru_hole oval (at 142.01 116.49) (size 1.65 1.65) (drill 1) (layers "*.Cu" "*.Mask") (remove_unused_layers no) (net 1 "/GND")
   (thermal_bridge_angle 45))
  (pad "120" thru_hole oval (at 144.55 116.49) (size 1.65 1.65) (drill 1) (layers "*.Cu" "*.Mask") (remove_unused_layers no) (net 1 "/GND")
   (thermal_bridge_angle 45)))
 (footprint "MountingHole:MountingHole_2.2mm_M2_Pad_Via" (layer "F.Cu") (at 112.5 87.5)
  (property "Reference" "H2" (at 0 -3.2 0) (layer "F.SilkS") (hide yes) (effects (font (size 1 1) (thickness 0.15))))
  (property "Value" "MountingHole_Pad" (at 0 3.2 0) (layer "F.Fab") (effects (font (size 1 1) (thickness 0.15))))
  (pad "1" thru_hole circle (at -1.65 0) (size 0.7 0.7) (drill 0.4) (layers "*.Cu" "*.Mask") (remove_unused_layers no))
  (pad "1" thru_hole circle (at -1.166726 -1.166726) (size 0.7 0.7) (drill 0.4) (layers "*.Cu" "*.Mask") (remove_unused_layers no))
  (pad "1" thru_hole circle (at -1.166726 1.166726) (size 0.7 0.7) (drill 0.4) (layers "*.Cu" "*.Mask") (remove_unused_layers no))
  (pad "1" thru_hole circle (at 0 -1.65) (size 0.7 0.7) (drill 0.4) (layers "*.Cu" "*.Mask") (remove_unused_layers no))
  (pad "1" thru_hole circle (at 0 0) (size 4.4 4.4) (drill 2.2) (layers "*.Cu" "*.Mask") (remove_unused_layers no))
  (pad "1" thru_hole circle (at 0 1.65) (size 0.7 0.7) (drill 0.4) (layers "*.Cu" "*.Mask") (remove_unused_layers no))
  (pad "1" thru_hole circle (at 1.166726 -1.166726) (size 0.7 0.7) (drill 0.4) (layers "*.Cu" "*.Mask") (remove_unused_layers no))
  (pad "1" thru_hole circle (at 1.166726 1.166726) (size 0.7 0.7) (drill 0.4) (layers "*.Cu" "*.Mask") (remove_unused_layers no))
  (pad "1" thru_hole circle (at 1.65 0) (size 0.7 0.7) (drill 0.4) (layers "*.Cu" "*.Mask") (remove_unused_layers no)))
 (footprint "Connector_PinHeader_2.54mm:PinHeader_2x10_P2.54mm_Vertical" (layer "F.Cu") (at 124.23 111.41 180)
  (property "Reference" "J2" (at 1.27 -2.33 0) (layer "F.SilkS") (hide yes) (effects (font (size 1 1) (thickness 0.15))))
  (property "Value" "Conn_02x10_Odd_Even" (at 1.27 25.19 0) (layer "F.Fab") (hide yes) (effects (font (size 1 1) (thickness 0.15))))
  (pad "1" thru_hole rect (at 0 0 180) (size 1.7 1.7) (drill 1) (layers "*.Cu" "*.Mask") (remove_unused_layers no) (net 1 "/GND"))
  (pad "2" thru_hole oval (at 2.54 0 180) (size 1.7 1.7) (drill 1) (layers "*.Cu" "*.Mask") (remove_unused_layers no) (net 1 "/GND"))
  (pad "3" thru_hole oval (at 0 2.54 180) (size 1.7 1.7) (drill 1) (layers "*.Cu" "*.Mask") (remove_unused_layers no) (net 2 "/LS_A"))
  (pad "4" thru_hole oval (at 2.54 2.54 180) (size 1.7 1.7) (drill 1) (layers "*.Cu" "*.Mask") (remove_unused_layers no) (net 13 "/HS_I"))
  (pad "5" thru_hole oval (at 0 5.08 180) (size 1.7 1.7) (drill 1) (layers "*.Cu" "*.Mask") (remove_unused_layers no) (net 3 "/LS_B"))
  (pad "6" thru_hole oval (at 2.54 5.08 180) (size 1.7 1.7) (drill 1) (layers "*.Cu" "*.Mask") (remove_unused_layers no) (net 12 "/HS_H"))
  (pad "7" thru_hole oval (at 0 7.62 180) (size 1.7 1.7) (drill 1) (layers "*.Cu" "*.Mask") (remove_unused_layers no) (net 4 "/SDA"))
  (pad "8" thru_hole oval (at 2.54 7.62 180) (size 1.7 1.7) (drill 1) (layers "*.Cu" "*.Mask") (remove_unused_layers no) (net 1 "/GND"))
  (pad "9" thru_hole oval (at 0 10.16 180) (size 1.7 1.7) (drill 1) (layers "*.Cu" "*.Mask") (remove_unused_layers no) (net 5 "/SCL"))
  (pad "10" thru_hole oval (at 2.54 10.16 180) (size 1.7 1.7) (drill 1) (layers "*.Cu" "*.Mask") (remove_unused_layers no) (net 11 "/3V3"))
  (pad "11" thru_hole oval (at 0 12.7 180) (size 1.7 1.7) (drill 1) (layers "*.Cu" "*.Mask") (remove_unused_layers no) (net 1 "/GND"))
  (pad "12" thru_hole oval (at 2.54 12.7 180) (size 1.7 1.7) (drill 1) (layers "*.Cu" "*.Mask") (remove_unused_layers no) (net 11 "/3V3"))
  (pad "13" thru_hole oval (at 0 15.24 180) (size 1.7 1.7) (drill 1) (layers "*.Cu" "*.Mask") (remove_unused_layers no) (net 6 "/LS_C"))
  (pad "14" thru_hole oval (at 2.54 15.24 180) (size 1.7 1.7) (drill 1) (layers "*.Cu" "*.Mask") (remove_unused_layers no) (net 1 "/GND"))
  (pad "15" thru_hole oval (at 0 17.78 180) (size 1.7 1.7) (drill 1) (layers "*.Cu" "*.Mask") (remove_unused_layers no) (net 7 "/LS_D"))
  (pad "16" thru_hole oval (at 2.54 17.78 180) (size 1.7 1.7) (drill 1) (layers "*.Cu" "*.Mask") (remove_unused_layers no) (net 10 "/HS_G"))
  (pad "17" thru_hole oval (at 0 20.32 180) (size 1.7 1.7) (drill 1) (layers "*.Cu" "*.Mask") (remove_unused_layers no) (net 8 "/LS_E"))
  (pad "18" thru_hole oval (at 2.54 20.32 180) (size 1.7 1.7) (drill 1) (layers "*.Cu" "*.Mask") (remove_unused_layers no) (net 9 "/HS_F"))
  (pad "19" thru_hole oval (at 0 22.86 180) (size 1.7 1.7) (drill 1) (layers "*.Cu" "*.Mask") (remove_unused_layers no) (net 1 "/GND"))
  (pad "20" thru_hole oval (at 2.54 22.86 180) (size 1.7 1.7) (drill 1) (layers "*.Cu" "*.Mask") (remove_unused_layers no) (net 1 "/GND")))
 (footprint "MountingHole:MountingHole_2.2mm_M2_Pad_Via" (layer "F.Cu") (at 112.5 112.5)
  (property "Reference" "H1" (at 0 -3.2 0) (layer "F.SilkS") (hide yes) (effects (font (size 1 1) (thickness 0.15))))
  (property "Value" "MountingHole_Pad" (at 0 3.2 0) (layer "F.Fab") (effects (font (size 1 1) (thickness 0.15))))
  (pad "1" thru_hole circle (at -1.65 0) (size 0.7 0.7) (drill 0.4) (layers "*.Cu" "*.Mask") (remove_unused_layers no))
  (pad "1" thru_hole circle (at -1.166726 -1.166726) (size 0.7 0.7) (drill 0.4) (layers "*.Cu" "*.Mask") (remove_unused_layers no))
  (pad "1" thru_hole circle (at -1.166726 1.166726) (size 0.7 0.7) (drill 0.4) (layers "*.Cu" "*.Mask") (remove_unused_layers no))
  (pad "1" thru_hole circle (at 0 -1.65) (size 0.7 0.7) (drill 0.4) (layers "*.Cu" "*.Mask") (remove_unused_layers no))
  (pad "1" thru_hole circle (at 0 0) (size 4.4 4.4) (drill 2.2) (layers "*.Cu" "*.Mask") (remove_unused_layers no))
  (pad "1" thru_hole circle (at 0 1.65) (size 0.7 0.7) (drill 0.4) (layers "*.Cu" "*.Mask") (remove_unused_layers no))
  (pad "1" thru_hole circle (at 1.166726 -1.166726) (size 0.7 0.7) (drill 0.4) (layers "*.Cu" "*.Mask") (remove_unused_layers no))
  (pad "1" thru_hole circle (at 1.166726 1.166726) (size 0.7 0.7) (drill 0.4) (layers "*.Cu" "*.Mask") (remove_unused_layers no))
  (pad "1" thru_hole circle (at 1.65 0) (size 0.7 0.7) (drill 0.4) (layers "*.Cu" "*.Mask") (remove_unused_layers no)))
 (gr_arc (start 100 91.33975) (mid 100.133975 90.83975) (end 100.5 90.473725) (stroke (width 0.05) (type default)) (layer "Edge.Cuts"))
 (gr_line (start 100 93.75) (end 100 91.33975) (stroke (width 0.05) (type default)) (layer "Edge.Cuts"))
 (gr_arc (start 100 106.25) (mid 100.073223 106.073223) (end 100.25 106) (stroke (width 0.1) (type default)) (layer "Edge.Cuts"))
 (gr_line (start 100 108.660243) (end 100 106.25) (stroke (width 0.05) (type default)) (layer "Edge.Cuts"))
 (gr_arc (start 100.25 94) (mid 100.073223 93.926777) (end 100 93.75) (stroke (width 0.1) (type default)) (layer "Edge.Cuts"))
 (gr_line (start 100.5 90.473725) (end 115.499995 81.813472) (stroke (width 0.05) (type default)) (layer "Edge.Cuts"))
 (gr_arc (start 100.5 109.526269) (mid 100.133975 109.160243) (end 100 108.660243) (stroke (width 0.05) (type default)) (layer "Edge.Cuts"))
 (gr_arc (start 115.499995 81.813472) (mid 115.999995 81.679497) (end 116.499995 81.813472) (stroke (width 0.05) (type default))
  (layer "Edge.Cuts"))
 (gr_line (start 115.499995 118.186522) (end 100.5 109.526269) (stroke (width 0.05) (type default)) (layer "Edge.Cuts"))
 (gr_line (start 116.499995 81.813472) (end 148 81.813472) (stroke (width 0.05) (type default)) (layer "Edge.Cuts"))
 (gr_arc (start 116.499995 118.186522) (mid 115.999995 118.320497) (end 115.499995 118.186522) (stroke (width 0.05) (type default))
  (layer "Edge.Cuts"))
 (gr_line (start 148 81.813472) (end 148 118.186522) (stroke (width 0.05) (type default)) (layer "Edge.Cuts"))
 (gr_line (start 148 118.186522) (end 116.499995 118.186522) (stroke (width 0.05) (type default)) (layer "Edge.Cuts"))
 (segment (start 111.99 103.8) (end 120.32 112.13) (width 0.25) (layer "F.Cu") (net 1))
 (segment (start 113.64 96.6) (end 100.5 96.6) (width 0.25) (layer "F.Cu") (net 1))
 (segment (start 121.69 88.55) (end 124.23 88.55) (width 0.25) (layer "F.Cu") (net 1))
 (segment (start 121.69 103.79) (end 119.3 101.4) (width 0.25) (layer "F.Cu") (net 1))
 (segment (start 118.86 99) (end 100.5 99) (width 0.25) (layer "F.Cu") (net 1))
 (segment (start 121.69 116.49) (end 144.55 116.49) (width 0.8) (layer "F.Cu") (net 1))
 (segment (start 120.97 112.13) (end 121.69 111.41) (width 0.25) (layer "F.Cu") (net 1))
 (segment (start 121.69 96.17) (end 118.86 99) (width 0.25) (layer "F.Cu") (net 1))
 (segment (start 121.69 88.55) (end 113.64 96.6) (width 0.25) (layer "F.Cu") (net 1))
 (segment (start 100.5 103.8) (end 111.99 103.8) (width 0.25) (layer "F.Cu") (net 1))
 (segment (start 119.3 101.4) (end 100.5 101.4) (width 0.25) (layer "F.Cu") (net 1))
 (segment (start 121.69 111.41) (end 124.23 111.41) (width 0.25) (layer "F.Cu") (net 1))
 (segment (start 122.5 102.52) (end 125.5 102.52) (width 0.25) (layer "F.Cu") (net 1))
 (segment (start 121.69 103.79) (end 122.5 102.52) (width 0.25) (layer "F.Cu") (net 1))
 (segment (start 120.32 112.13) (end 120.97 112.13) (width 0.25) (layer "F.Cu") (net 1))
 (via (at 125.5 102.52) (size 0.6) (drill 0.3) (layers "F.Cu" "B.Cu") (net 1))
 (segment (start 121.69 96.17) (end 122.5 97.45) (width 0.25) (layer "B.Cu") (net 1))
 (segment (start 125.5 112.68) (end 125.5 116.49) (width 0.25) (layer "B.Cu") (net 1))
 (segment (start 120.4 97.41) (end 118.41 99.4) (width 0.25) (layer "B.Cu") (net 1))
 (segment (start 112.45 103.4) (end 100.5 103.4) (width 0.25) (layer "B.Cu") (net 1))
 (segment (start 121.69 111.41) (end 120.62 111.41) (width 0.25) (layer "B.Cu") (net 1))
 (segment (start 124.23 98.71) (end 122.93 97.41) (width 0.25) (layer "B.Cu") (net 1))
 (segment (start 120.54 111.49) (end 112.45 103.4) (width 0.25) (layer "B.Cu") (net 1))
 (segment (start 119.36 88.55) (end 111.71 96.2) (width 0.25) (layer "B.Cu") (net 1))
 (segment (start 122.5 97.45) (end 125.5 97.45) (width 0.25) (layer "B.Cu") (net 1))
 (segment (start 120.62 111.41) (end 120.54 111.49) (width 0.25) (layer "B.Cu") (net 1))
 (segment (start 124.23 111.41) (end 125.5 112.68) (width 0.25) (layer "B.Cu") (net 1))
 (segment (start 125.5 116.49) (end 121.69 116.49) (width 0.25) (layer "B.Cu") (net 1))
 (segment (start 111.71 96.2) (end 100.5 96.2) (width 0.25) (layer "B.Cu") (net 1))
 (segment (start 124.23 88.55) (end 125.5 88.55) (width 0.25) (layer "B.Cu") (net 1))
 (segment (start 125.5 88.55) (end 125.5 116.49) (width 0.25) (layer "B.Cu") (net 1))
 (segment (start 122.93 97.41) (end 120.4 97.41) (width 0.25) (layer "B.Cu") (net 1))
 (segment (start 124.23 98.71) (end 125.5 98.71) (width 0.25) (layer "B.Cu") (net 1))
 (segment (start 118.41 99.4) (end 100.9 99.4) (width 0.25) (layer "B.Cu") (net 1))
 (segment (start 121.69 88.55) (end 119.36 88.55) (width 0.25) (layer "B.Cu") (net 1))
 (segment (start 123.055 107.695) (end 120.735 107.695) (width 0.25) (layer "B.Cu") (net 2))
 (segment (start 120.735 107.695) (end 120.73 107.7) (width 0.25) (layer "B.Cu") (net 2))
 (segment (start 124.23 108.87) (end 123.055 107.695) (width 0.25) (layer "B.Cu") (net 2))
 (segment (start 115.63 102.6) (end 100.9 102.6) (width 0.25) (layer "B.Cu") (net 2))
 (segment (start 120.73 107.7) (end 115.63 102.6) (width 0.25) (layer "B.Cu") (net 2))
 (segment (start 124.23 106.33) (end 122.94 105.04) (width 0.25) (layer "B.Cu") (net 3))
 (segment (start 120.42 105.04) (end 117.18 101.8) (width 0.25) (layer "B.Cu") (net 3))
 (segment (start 117.18 101.8) (end 100.9 101.8) (width 0.25) (layer "B.Cu") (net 3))
 (segment (start 122.94 105.04) (end 120.42 105.04) (width 0.25) (layer "B.Cu") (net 3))
 (segment (start 122.44 102.48) (end 120.96 102.48) (width 0.25) (layer "B.Cu") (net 4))
 (segment (start 123.75 103.79) (end 122.44 102.48) (width 0.25) (layer "B.Cu") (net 4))
 (segment (start 124.23 103.79) (end 123.75 103.79) (width 0.25) (layer "B.Cu") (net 4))
 (segment (start 120.96 102.48) (end 119.48 101) (width 0.25) (layer "B.Cu") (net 4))
 (segment (start 119.48 101) (end 100.9 101) (width 0.25) (layer "B.Cu") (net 4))
 (segment (start 124.23 101.25) (end 122.94 99.96) (width 0.25) (layer "B.Cu") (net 5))
 (segment (start 122.94 99.96) (end 103.5 99.96) (width 0.25) (layer "B.Cu") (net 5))
 (segment (start 103.26 100.2) (end 100.9 100.2) (width 0.25) (layer "B.Cu") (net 5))
 (segment (start 103.5 99.96) (end 103.26 100.2) (width 0.25) (layer "B.Cu") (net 5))
 (segment (start 124.23 95.92) (end 123.23 94.92) (width 0.25) (layer "B.Cu") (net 6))
 (segment (start 116.25 98.6) (end 100.9 98.6) (width 0.25) (layer "B.Cu") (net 6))
 (segment (start 123.23 94.92) (end 119.93 94.92) (width 0.25) (layer "B.Cu") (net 6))
 (segment (start 119.93 94.92) (end 116.25 98.6) (width 0.25) (layer "B.Cu") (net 6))
 (segment (start 124.23 96.17) (end 124.23 95.92) (width 0.25) (layer "B.Cu") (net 6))
 (segment (start 114.52 97.8) (end 100.9 97.8) (width 0.25) (layer "B.Cu") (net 7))
 (segment (start 122.94 92.34) (end 119.98 92.34) (width 0.25) (layer "B.Cu") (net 7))
 (segment (start 119.98 92.34) (end 114.52 97.8) (width 0.25) (layer "B.Cu") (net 7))
 (segment (start 124.23 93.63) (end 122.94 92.34) (width 0.25) (layer "B.Cu") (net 7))
 (segment (start 113.28 97) (end 100.5 97) (width 0.25) (layer "B.Cu") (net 8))
 (segment (start 124.23 91.09) (end 122.99 89.85) (width 0.25) (layer "B.Cu") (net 8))
 (segment (start 120.43 89.85) (end 113.28 97) (width 0.25) (layer "B.Cu") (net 8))
 (segment (start 122.99 89.85) (end 120.43 89.85) (width 0.25) (layer "B.Cu") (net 8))
 (segment (start 115.38 97.4) (end 100.9 97.4) (width 0.25) (layer "F.Cu") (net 9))
 (segment (start 121.69 91.09) (end 115.38 97.4) (width 0.25) (layer "F.Cu") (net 9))
 (segment (start 117.12 98.2) (end 100.9 98.2) (width 0.25) (layer "F.Cu") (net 10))
 (segment (start 121.69 93.63) (end 117.12 98.2) (width 0.25) (layer "F.Cu") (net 10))
 (segment (start 133.12 100) (end 133.12 83.47) (width 0.25) (layer "F.Cu") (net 11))
 (segment (start 120.6 99.8) (end 100.9 99.8) (width 0.25) (layer "F.Cu") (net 11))
 (segment (start 121.69 100) (end 133.12 100) (width 0.25) (layer "F.Cu") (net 11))
 (segment (start 100.9 99.8) (end 100.9 100.6) (width 0.25) (layer "F.Cu") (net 11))
 (segment (start 133.12 83.47) (end 121.69 83.47) (width 0.25) (layer "F.Cu") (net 11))
 (segment (start 121.69 98.71) (end 120.6 99.8) (width 0.25) (layer "F.Cu") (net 11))
 (segment (start 121.69 83.47) (end 144.55 83.47) (width 0.8) (layer "F.Cu") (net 11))
 (segment (start 100.9 100.6) (end 121.04 100.6) (width 0.25) (layer "F.Cu") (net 11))
 (segment (start 121.69 101.25) (end 121.69 100) (width 0.25) (layer "F.Cu") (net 11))
 (segment (start 121.69 106.33) (end 120.38 106.33) (width 0.25) (layer "F.Cu") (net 12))
 (segment (start 116.25 102.2) (end 100.9 102.2) (width 0.25) (layer "F.Cu") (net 12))
 (segment (start 120.38 106.33) (end 116.25 102.2) (width 0.25) (layer "F.Cu") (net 12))
 (segment (start 121.69 108.87) (end 120.28 108.87) (width 0.25) (layer "F.Cu") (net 13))
 (segment (start 120.28 108.87) (end 114.41 103) (width 0.25) (layer "F.Cu") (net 13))
 (segment (start 114.41 103) (end 100.9 103) (width 0.25) (layer "F.Cu") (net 13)))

